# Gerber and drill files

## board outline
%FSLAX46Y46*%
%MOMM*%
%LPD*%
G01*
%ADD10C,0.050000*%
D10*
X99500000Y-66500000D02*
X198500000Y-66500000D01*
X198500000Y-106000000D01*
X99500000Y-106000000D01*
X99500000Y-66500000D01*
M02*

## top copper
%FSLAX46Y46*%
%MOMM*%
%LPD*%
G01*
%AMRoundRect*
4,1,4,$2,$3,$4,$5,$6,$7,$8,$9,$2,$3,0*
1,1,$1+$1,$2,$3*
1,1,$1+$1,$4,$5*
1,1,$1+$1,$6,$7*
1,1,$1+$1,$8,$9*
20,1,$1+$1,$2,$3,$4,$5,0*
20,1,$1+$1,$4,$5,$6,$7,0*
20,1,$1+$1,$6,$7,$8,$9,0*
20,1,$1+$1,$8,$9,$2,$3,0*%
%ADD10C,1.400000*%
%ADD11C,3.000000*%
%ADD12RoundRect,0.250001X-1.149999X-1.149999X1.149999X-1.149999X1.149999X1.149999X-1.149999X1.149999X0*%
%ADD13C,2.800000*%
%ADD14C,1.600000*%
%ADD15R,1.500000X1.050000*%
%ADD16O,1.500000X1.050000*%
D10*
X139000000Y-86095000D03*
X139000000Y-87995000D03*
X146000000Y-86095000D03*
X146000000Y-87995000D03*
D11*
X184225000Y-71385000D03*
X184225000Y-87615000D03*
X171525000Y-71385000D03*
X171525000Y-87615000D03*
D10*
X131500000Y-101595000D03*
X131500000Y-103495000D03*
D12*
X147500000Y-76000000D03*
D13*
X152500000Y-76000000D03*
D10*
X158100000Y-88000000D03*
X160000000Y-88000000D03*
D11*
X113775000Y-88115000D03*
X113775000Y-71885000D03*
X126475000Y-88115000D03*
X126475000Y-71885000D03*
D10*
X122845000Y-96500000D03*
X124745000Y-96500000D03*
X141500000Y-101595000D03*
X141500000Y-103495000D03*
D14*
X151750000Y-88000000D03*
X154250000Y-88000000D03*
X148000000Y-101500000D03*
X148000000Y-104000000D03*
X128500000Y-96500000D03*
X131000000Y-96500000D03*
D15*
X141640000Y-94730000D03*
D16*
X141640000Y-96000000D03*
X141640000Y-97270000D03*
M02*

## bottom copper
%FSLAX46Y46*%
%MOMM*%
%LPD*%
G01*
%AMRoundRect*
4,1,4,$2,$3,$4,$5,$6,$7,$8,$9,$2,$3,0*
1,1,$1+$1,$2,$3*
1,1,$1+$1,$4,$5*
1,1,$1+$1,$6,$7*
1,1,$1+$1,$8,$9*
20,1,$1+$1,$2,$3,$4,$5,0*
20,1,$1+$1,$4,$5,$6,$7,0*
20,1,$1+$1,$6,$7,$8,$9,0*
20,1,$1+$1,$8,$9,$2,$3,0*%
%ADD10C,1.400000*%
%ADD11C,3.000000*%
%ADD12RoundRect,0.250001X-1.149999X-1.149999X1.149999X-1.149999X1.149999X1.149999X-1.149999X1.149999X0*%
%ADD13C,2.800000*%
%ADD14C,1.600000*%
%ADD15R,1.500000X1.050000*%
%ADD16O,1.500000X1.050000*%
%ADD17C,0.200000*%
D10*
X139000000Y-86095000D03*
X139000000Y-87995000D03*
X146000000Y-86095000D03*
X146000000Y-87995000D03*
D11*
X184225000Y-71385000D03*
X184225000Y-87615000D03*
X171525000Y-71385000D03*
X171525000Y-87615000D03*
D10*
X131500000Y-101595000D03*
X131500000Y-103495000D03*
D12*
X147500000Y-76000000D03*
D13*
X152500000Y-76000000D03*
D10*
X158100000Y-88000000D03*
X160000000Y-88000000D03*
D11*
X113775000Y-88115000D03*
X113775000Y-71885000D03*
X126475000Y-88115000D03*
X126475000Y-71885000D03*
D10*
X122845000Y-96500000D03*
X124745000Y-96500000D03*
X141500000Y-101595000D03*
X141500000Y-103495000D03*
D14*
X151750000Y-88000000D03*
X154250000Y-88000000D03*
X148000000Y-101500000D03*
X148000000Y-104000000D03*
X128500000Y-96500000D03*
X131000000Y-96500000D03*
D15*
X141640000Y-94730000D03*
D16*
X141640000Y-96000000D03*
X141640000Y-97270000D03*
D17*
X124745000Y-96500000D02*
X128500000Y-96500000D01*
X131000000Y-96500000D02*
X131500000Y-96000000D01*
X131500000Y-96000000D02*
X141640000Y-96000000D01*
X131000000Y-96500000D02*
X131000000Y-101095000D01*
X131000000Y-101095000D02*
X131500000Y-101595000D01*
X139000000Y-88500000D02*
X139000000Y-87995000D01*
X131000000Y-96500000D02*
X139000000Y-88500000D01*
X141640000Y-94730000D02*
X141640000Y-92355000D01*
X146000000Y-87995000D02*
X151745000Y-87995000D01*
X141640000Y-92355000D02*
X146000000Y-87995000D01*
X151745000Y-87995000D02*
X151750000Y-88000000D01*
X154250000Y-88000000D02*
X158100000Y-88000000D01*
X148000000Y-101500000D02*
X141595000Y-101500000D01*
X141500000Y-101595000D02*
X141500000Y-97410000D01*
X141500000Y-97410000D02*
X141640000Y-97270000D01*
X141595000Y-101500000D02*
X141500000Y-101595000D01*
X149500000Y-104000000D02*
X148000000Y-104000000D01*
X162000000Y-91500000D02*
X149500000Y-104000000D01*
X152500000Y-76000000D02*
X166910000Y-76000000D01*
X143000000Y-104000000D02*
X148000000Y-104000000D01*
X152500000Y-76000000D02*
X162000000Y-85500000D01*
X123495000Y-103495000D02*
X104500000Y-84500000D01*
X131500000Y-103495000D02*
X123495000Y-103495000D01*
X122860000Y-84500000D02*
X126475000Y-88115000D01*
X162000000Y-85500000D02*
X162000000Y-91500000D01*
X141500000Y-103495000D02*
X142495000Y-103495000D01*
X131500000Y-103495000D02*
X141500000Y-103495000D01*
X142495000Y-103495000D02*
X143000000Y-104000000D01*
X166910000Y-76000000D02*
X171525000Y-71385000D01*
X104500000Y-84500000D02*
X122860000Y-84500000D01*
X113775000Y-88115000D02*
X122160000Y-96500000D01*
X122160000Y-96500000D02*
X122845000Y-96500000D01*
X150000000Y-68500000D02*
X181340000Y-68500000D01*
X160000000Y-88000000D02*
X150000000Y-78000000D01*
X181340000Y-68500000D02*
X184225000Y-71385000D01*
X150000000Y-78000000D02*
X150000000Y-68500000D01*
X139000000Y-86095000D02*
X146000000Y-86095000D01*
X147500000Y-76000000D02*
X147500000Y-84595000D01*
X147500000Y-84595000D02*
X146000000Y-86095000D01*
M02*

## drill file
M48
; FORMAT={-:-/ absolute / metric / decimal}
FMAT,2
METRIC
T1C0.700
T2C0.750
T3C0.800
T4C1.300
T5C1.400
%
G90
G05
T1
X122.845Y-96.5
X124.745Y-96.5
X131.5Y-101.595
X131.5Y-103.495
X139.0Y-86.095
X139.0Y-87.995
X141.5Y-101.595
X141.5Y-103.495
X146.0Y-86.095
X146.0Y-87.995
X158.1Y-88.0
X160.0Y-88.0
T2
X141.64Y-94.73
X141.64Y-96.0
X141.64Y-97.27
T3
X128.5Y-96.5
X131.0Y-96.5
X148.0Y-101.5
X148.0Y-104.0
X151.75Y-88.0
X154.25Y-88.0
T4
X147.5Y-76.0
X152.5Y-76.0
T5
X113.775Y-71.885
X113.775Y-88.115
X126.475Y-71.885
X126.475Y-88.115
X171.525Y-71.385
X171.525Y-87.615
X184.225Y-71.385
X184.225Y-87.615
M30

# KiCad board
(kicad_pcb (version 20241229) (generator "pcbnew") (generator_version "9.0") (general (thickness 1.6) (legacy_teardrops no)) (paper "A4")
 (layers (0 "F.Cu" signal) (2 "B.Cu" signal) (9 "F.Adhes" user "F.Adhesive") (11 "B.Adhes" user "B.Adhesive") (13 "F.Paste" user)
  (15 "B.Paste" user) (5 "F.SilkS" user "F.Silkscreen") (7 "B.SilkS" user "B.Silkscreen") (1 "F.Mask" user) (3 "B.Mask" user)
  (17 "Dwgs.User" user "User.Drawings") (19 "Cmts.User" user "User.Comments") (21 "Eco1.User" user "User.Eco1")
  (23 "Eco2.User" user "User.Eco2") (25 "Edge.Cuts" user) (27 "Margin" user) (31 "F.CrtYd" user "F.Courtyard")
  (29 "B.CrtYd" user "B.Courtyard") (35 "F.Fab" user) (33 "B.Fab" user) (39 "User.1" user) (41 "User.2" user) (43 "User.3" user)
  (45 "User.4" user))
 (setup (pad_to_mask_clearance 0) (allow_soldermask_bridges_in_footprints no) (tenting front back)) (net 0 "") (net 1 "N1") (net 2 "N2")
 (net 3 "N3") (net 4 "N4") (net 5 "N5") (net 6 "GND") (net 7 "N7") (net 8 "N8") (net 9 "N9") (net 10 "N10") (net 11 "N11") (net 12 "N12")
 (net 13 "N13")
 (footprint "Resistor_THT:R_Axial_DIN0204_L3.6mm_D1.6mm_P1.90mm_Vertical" (layer "F.Cu") (at 139 86.095 -90)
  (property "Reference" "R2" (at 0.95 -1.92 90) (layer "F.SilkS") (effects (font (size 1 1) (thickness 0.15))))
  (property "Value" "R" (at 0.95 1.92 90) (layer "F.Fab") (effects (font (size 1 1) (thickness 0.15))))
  (pad "1" thru_hole circle (at 0 0 270) (size 1.4 1.4) (drill 0.7) (layers "*.Cu" "*.Mask") (remove_unused_layers no) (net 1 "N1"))
  (pad "2" thru_hole circle (at 1.9 0 270) (size 1.4 1.4) (drill 0.7) (layers "*.Cu" "*.Mask") (remove_unused_layers no) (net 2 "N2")))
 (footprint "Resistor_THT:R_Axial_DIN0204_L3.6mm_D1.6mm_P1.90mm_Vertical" (layer "F.Cu") (at 146 86.095 -90)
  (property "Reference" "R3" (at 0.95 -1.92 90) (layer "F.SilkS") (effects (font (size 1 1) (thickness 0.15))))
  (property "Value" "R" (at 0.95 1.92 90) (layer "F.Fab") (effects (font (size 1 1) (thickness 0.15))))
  (pad "1" thru_hole circle (at 0 0 270) (size 1.4 1.4) (drill 0.7) (layers "*.Cu" "*.Mask") (remove_unused_layers no) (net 1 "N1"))
  (pad "2" thru_hole circle (at 1.9 0 270) (size 1.4 1.4) (drill 0.7) (layers "*.Cu" "*.Mask") (remove_unused_layers no) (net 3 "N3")))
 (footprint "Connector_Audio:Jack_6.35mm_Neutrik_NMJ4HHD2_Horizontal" (layer "F.Cu") (at 171.525 71.385)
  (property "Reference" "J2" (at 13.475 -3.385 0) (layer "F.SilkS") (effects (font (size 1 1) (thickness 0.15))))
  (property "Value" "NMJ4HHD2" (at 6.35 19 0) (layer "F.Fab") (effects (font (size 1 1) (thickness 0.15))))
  (pad "S" thru_hole circle (at 12.7 0) (size 3 3) (drill 1.4) (layers "*.Cu" "*.Mask") (remove_unused_layers no) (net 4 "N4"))
  (pad "SN" thru_hole circle (at 12.7 16.23) (size 3 3) (drill 1.4) (layers "*.Cu" "*.Mask") (remove_unused_layers no) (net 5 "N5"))
  (pad "T" thru_hole circle (at 0 0) (size 3 3) (drill 1.4) (layers "*.Cu" "*.Mask") (remove_unused_layers no) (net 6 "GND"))
  (pad "TN" thru_hole circle (at 0 16.23) (size 3 3) (drill 1.4) (layers "*.Cu" "*.Mask") (remove_unused_layers no) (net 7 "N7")))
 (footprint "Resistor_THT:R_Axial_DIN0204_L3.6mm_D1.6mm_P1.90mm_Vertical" (layer "F.Cu") (at 131.5 101.595 -90)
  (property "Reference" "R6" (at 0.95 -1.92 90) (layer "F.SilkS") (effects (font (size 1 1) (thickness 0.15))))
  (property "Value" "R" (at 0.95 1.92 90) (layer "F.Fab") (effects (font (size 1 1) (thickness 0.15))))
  (pad "1" thru_hole circle (at 0 0 270) (size 1.4 1.4) (drill 0.7) (layers "*.Cu" "*.Mask") (remove_unused_layers no) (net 2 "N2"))
  (pad "2" thru_hole circle (at 1.9 0 270) (size 1.4 1.4) (drill 0.7) (layers "*.Cu" "*.Mask") (remove_unused_layers no) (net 6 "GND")))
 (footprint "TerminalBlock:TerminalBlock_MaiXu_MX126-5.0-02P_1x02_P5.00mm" (layer "F.Cu") (at 147.5 76)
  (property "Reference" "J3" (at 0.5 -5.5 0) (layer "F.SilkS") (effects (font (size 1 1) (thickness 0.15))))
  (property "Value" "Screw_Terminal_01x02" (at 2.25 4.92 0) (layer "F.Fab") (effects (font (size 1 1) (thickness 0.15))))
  (pad "1" thru_hole roundrect (at 0 0) (size 2.8 2.8) (drill 1.3) (layers "*.Cu" "*.Mask") (remove_unused_layers no)
   (roundrect_rratio 0.089286) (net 1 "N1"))
  (pad "2" thru_hole circle (at 5 0) (size 2.8 2.8) (drill 1.3) (layers "*.Cu" "*.Mask") (remove_unused_layers no) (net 6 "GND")))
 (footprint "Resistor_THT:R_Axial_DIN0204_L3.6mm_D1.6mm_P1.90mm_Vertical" (layer "F.Cu") (at 158.1 88)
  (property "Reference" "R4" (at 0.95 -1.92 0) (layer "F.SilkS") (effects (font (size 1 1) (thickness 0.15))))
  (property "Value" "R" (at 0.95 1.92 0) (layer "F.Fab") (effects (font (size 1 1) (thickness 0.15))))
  (pad "1" thru_hole circle (at 0 0) (size 1.4 1.4) (drill 0.7) (layers "*.Cu" "*.Mask") (remove_unused_layers no) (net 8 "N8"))
  (pad "2" thru_hole circle (at 1.9 0) (size 1.4 1.4) (drill 0.7) (layers "*.Cu" "*.Mask") (remove_unused_layers no) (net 4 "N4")))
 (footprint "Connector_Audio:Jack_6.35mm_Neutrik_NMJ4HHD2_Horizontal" (layer "F.Cu") (at 126.475 88.115 180)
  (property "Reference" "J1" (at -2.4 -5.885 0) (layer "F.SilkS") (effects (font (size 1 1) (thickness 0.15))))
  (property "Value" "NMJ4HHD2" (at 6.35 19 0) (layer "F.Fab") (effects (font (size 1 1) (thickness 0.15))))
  (pad "S" thru_hole circle (at 12.7 0 180) (size 3 3) (drill 1.4) (layers "*.Cu" "*.Mask") (remove_unused_layers no) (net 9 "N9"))
  (pad "SN" thru_hole circle (at 12.7 16.23 180) (size 3 3) (drill 1.4) (layers "*.Cu" "*.Mask") (remove_unused_layers no) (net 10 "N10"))
  (pad "T" thru_hole circle (at 0 0 180) (size 3 3) (drill 1.4) (layers "*.Cu" "*.Mask") (remove_unused_layers no) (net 6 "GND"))
  (pad "TN" thru_hole circle (at 0 16.23 180) (size 3 3) (drill 1.4) (layers "*.Cu" "*.Mask") (remove_unused_layers no) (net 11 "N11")))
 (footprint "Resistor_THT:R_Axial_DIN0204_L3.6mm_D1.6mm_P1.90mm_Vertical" (layer "F.Cu") (at 122.845 96.5)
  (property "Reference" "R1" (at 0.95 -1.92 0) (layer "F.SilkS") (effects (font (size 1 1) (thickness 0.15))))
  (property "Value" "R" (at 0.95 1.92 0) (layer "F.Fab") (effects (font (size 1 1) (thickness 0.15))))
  (pad "1" thru_hole circle (at 0 0) (size 1.4 1.4) (drill 0.7) (layers "*.Cu" "*.Mask") (remove_unused_layers no) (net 9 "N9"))
  (pad "2" thru_hole circle (at 1.9 0) (size 1.4 1.4) (drill 0.7) (layers "*.Cu" "*.Mask") (remove_unused_layers no) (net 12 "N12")))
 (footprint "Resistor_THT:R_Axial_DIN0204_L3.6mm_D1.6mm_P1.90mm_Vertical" (layer "F.Cu") (at 141.5 101.595 -90)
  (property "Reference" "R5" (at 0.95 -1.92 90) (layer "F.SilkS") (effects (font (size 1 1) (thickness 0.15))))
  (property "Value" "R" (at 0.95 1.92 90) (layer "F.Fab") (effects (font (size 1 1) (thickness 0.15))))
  (pad "1" thru_hole circle (at 0 0 270) (size 1.4 1.4) (drill 0.7) (layers "*.Cu" "*.Mask") (remove_unused_layers no) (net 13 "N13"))
  (pad "2" thru_hole circle (at 1.9 0 270) (size 1.4 1.4) (drill 0.7) (layers "*.Cu" "*.Mask") (remove_unused_layers no) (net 6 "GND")))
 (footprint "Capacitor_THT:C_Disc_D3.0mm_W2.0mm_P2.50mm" (layer "F.Cu") (at 151.75 88)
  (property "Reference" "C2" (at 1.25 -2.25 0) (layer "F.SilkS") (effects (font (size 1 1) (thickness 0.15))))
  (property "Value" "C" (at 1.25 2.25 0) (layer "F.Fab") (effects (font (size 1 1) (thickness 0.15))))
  (pad "1" thru_hole circle (at 0 0) (size 1.6 1.6) (drill 0.8) (layers "*.Cu" "*.Mask") (remove_unused_layers no) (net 3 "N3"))
  (pad "2" thru_hole circle (at 2.5 0) (size 1.6 1.6) (drill 0.8) (layers "*.Cu" "*.Mask") (remove_unused_layers no) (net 8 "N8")))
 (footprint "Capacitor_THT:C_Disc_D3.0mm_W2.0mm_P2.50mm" (layer "F.Cu") (at 148 101.5 -90)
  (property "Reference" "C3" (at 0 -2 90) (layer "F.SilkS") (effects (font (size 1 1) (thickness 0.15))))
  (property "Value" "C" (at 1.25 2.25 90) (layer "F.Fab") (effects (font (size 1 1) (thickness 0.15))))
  (pad "1" thru_hole circle (at 0 0 270) (size 1.6 1.6) (drill 0.8) (layers "*.Cu" "*.Mask") (remove_unused_layers no) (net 13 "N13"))
  (pad "2" thru_hole circle (at 2.5 0 270) (size 1.6 1.6) (drill 0.8) (layers "*.Cu" "*.Mask") (remove_unused_layers no) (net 6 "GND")))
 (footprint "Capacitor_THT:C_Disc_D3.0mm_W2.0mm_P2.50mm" (layer "F.Cu") (at 128.5 96.5)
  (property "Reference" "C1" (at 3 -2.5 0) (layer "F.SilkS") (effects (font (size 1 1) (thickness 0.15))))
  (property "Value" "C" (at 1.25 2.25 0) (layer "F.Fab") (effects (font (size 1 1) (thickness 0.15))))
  (pad "1" thru_hole circle (at 0 0) (size 1.6 1.6) (drill 0.8) (layers "*.Cu" "*.Mask") (remove_unused_layers no) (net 12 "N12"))
  (pad "2" thru_hole circle (at 2.5 0) (size 1.6 1.6) (drill 0.8) (layers "*.Cu" "*.Mask") (remove_unused_layers no) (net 2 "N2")))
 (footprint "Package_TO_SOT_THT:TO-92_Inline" (layer "F.Cu") (at 141.64 94.73 -90)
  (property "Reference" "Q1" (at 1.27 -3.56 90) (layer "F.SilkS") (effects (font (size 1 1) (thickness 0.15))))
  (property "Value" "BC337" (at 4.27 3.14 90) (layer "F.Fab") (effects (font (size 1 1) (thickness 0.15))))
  (pad "1" thru_hole rect (at 0 0 270) (size 1.05 1.5) (drill 0.75) (layers "*.Cu" "*.Mask") (remove_unused_layers no) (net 3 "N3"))
  (pad "2" thru_hole oval (at 1.27 0 270) (size 1.05 1.5) (drill 0.75) (layers "*.Cu" "*.Mask") (remove_unused_layers no) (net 2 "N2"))
  (pad "3" thru_hole oval (at 2.54 0 270) (size 1.05 1.5) (drill 0.75) (layers "*.Cu" "*.Mask") (remove_unused_layers no) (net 13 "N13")))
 (gr_rect (start 99.5 66.5) (end 198.5 106) (stroke (width 0.05) (type default)) (fill no) (layer "Edge.Cuts"))
 (segment (start 124.745 96.5) (end 128.5 96.5) (width 0.2) (layer "B.Cu") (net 12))
 (segment (start 131 96.5) (end 131.5 96) (width 0.2) (layer "B.Cu") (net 2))
 (segment (start 131.5 96) (end 141.64 96) (width 0.2) (layer "B.Cu") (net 2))
 (segment (start 131 96.5) (end 131 101.095) (width 0.2) (layer "B.Cu") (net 2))
 (segment (start 131 101.095) (end 131.5 101.595) (width 0.2) (layer "B.Cu") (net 2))
 (segment (start 139 88.5) (end 139 87.995) (width 0.2) (layer "B.Cu") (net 2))
 (segment (start 131 96.5) (end 139 88.5) (width 0.2) (layer "B.Cu") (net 2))
 (segment (start 141.64 94.73) (end 141.64 92.355) (width 0.2) (layer "B.Cu") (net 3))
 (segment (start 146 87.995) (end 151.745 87.995) (width 0.2) (layer "B.Cu") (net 3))
 (segment (start 141.64 92.355) (end 146 87.995) (width 0.2) (layer "B.Cu") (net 3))
 (segment (start 151.745 87.995) (end 151.75 88) (width 0.2) (layer "B.Cu") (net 3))
 (segment (start 154.25 88) (end 158.1 88) (width 0.2) (layer "B.Cu") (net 8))
 (segment (start 148 101.5) (end 141.595 101.5) (width 0.2) (layer "B.Cu") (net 13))
 (segment (start 141.5 101.595) (end 141.5 97.41) (width 0.2) (layer "B.Cu") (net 13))
 (segment (start 141.5 97.41) (end 141.64 97.27) (width 0.2) (layer "B.Cu") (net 13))
 (segment (start 141.595 101.5) (end 141.5 101.595) (width 0.2) (layer "B.Cu") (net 13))
 (segment (start 149.5 104) (end 148 104) (width 0.2) (layer "B.Cu") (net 6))
 (segment (start 162 91.5) (end 149.5 104) (width 0.2) (layer "B.Cu") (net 6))
 (segment (start 152.5 76) (end 166.91 76) (width 0.2) (layer "B.Cu") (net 6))
 (segment (start 143 104) (end 148 104) (width 0.2) (layer "B.Cu") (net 6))
 (segment (start 152.5 76) (end 162 85.5) (width 0.2) (layer "B.Cu") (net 6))
 (segment (start 123.495 103.495) (end 104.5 84.5) (width 0.2) (layer "B.Cu") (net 6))
 (segment (start 131.5 103.495) (end 123.495 103.495) (width 0.2) (layer "B.Cu") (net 6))
 (segment (start 122.86 84.5) (end 126.475 88.115) (width 0.2) (layer "B.Cu") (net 6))
 (segment (start 162 85.5) (end 162 91.5) (width 0.2) (layer "B.Cu") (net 6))
 (segment (start 141.5 103.495) (end 142.495 103.495) (width 0.2) (layer "B.Cu") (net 6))
 (segment (start 131.5 103.495) (end 141.5 103.495) (width 0.2) (layer "B.Cu") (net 6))
 (segment (start 142.495 103.495) (end 143 104) (width 0.2) (layer "B.Cu") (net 6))
 (segment (start 166.91 76) (end 171.525 71.385) (width 0.2) (layer "B.Cu") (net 6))
 (segment (start 104.5 84.5) (end 122.86 84.5) (width 0.2) (layer "B.Cu") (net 6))
 (segment (start 113.775 88.115) (end 122.16 96.5) (width 0.2) (layer "B.Cu") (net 9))
 (segment (start 122.16 96.5) (end 122.845 96.5) (width 0.2) (layer "B.Cu") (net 9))
 (segment (start 150 68.5) (end 181.34 68.5) (width 0.2) (layer "B.Cu") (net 4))
 (segment (start 160 88) (end 150 78) (width 0.2) (layer "B.Cu") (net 4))
 (segment (start 181.34 68.5) (end 184.225 71.385) (width 0.2) (layer "B.Cu") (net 4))
 (segment (start 150 78) (end 150 68.5) (width 0.2) (layer "B.Cu") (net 4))
 (segment (start 139 86.095) (end 146 86.095) (width 0.2) (layer "B.Cu") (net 1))
 (segment (start 147.5 76) (end 147.5 84.595) (width 0.2) (layer "B.Cu") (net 1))
 (segment (start 147.5 84.595) (end 146 86.095) (width 0.2) (layer "B.Cu") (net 1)))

